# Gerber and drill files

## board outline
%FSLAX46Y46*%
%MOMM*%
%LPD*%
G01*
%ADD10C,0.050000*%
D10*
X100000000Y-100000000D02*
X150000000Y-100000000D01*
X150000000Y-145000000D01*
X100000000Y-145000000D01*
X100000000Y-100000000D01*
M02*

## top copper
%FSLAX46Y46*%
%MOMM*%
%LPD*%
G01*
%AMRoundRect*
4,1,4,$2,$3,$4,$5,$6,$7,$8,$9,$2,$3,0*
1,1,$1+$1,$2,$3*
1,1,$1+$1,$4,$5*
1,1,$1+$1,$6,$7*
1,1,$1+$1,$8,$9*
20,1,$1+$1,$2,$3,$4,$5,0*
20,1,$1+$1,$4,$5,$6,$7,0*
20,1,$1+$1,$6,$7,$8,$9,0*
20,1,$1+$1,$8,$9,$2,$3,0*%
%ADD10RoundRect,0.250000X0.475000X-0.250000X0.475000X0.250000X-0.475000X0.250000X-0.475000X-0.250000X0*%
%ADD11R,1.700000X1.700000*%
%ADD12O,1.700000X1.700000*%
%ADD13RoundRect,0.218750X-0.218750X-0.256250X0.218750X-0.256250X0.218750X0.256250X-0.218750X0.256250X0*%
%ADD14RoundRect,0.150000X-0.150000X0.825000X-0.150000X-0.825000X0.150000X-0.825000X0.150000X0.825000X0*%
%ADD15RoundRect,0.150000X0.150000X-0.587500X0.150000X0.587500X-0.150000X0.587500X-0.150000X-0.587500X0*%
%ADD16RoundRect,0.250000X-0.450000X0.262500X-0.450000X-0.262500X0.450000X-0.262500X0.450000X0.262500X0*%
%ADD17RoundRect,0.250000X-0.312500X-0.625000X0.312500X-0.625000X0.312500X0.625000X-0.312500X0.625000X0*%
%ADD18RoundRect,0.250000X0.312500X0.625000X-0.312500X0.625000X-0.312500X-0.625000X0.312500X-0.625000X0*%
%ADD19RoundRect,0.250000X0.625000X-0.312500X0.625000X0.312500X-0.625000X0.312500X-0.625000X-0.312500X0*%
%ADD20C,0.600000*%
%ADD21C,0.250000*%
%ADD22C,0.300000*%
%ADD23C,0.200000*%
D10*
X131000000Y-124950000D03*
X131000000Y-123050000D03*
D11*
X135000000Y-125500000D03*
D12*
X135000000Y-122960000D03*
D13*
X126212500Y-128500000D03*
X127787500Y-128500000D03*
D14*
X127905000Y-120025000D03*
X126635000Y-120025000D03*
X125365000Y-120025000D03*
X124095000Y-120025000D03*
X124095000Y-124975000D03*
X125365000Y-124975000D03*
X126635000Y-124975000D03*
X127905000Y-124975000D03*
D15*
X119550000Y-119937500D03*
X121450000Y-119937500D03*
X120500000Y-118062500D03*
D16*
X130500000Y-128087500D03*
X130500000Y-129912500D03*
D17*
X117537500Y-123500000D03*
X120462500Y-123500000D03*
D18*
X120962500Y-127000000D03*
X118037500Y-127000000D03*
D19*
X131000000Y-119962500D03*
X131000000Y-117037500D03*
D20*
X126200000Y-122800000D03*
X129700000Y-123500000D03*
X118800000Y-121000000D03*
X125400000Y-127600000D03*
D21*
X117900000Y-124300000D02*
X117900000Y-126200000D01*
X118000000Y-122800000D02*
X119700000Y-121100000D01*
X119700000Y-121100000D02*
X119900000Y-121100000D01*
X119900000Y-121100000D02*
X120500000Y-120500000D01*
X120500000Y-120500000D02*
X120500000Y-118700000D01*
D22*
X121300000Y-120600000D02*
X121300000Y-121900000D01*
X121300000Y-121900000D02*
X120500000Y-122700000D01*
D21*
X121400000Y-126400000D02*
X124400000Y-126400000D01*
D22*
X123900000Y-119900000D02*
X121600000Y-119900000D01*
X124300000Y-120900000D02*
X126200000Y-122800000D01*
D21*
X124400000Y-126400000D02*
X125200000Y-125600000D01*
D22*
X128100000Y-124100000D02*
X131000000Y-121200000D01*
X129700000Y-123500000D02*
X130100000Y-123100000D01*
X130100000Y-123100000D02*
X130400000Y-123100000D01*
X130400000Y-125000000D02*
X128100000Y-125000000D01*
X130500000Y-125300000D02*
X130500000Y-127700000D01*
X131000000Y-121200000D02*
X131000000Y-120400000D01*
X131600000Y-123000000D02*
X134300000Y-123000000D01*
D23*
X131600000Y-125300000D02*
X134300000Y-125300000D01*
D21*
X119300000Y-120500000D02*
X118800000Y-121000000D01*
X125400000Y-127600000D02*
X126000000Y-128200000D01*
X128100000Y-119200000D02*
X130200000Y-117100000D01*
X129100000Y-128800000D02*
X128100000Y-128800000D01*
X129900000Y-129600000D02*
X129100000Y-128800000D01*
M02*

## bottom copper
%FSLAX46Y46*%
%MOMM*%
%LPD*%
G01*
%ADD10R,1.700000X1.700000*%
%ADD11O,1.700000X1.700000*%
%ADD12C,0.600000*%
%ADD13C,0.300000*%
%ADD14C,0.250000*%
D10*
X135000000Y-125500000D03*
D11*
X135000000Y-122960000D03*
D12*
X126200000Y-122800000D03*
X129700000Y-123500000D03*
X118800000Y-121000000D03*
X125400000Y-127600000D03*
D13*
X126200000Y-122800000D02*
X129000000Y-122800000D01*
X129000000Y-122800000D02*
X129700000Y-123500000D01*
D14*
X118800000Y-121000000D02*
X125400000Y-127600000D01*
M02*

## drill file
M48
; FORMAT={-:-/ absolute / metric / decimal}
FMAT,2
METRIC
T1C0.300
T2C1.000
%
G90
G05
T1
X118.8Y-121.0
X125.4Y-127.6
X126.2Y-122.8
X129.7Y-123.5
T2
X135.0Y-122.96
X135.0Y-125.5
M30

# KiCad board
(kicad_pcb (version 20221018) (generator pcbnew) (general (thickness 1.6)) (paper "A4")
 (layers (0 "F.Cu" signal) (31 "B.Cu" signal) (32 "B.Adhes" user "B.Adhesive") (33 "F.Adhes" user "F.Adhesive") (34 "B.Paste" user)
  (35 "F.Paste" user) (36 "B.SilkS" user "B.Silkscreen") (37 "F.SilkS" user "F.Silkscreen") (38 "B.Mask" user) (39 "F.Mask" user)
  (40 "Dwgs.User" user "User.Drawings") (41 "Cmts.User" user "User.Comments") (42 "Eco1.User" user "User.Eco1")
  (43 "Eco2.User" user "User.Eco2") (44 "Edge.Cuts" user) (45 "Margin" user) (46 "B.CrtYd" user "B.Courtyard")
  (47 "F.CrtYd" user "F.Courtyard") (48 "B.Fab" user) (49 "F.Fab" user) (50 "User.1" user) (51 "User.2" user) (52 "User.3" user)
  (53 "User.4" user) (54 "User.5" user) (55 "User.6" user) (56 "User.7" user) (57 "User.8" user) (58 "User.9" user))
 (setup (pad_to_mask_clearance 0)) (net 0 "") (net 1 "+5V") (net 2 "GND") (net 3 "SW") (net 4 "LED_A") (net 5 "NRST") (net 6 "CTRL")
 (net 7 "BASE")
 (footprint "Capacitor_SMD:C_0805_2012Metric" (layer "F.Cu") (at 131 124 90)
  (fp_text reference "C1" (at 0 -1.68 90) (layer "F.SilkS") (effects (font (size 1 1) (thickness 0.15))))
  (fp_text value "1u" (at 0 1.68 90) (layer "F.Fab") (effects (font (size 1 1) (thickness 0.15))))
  (pad "1" smd roundrect (at -0.95 0 90) (size 1 1.45) (layers "F.Cu" "F.Paste" "F.Mask") (roundrect_rratio 0.25) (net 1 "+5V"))
  (pad "2" smd roundrect (at 0.95 0 90) (size 1 1.45) (layers "F.Cu" "F.Paste" "F.Mask") (roundrect_rratio 0.25) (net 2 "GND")))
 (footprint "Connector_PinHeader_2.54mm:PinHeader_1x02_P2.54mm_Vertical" (layer "F.Cu") (at 135 125.5 180)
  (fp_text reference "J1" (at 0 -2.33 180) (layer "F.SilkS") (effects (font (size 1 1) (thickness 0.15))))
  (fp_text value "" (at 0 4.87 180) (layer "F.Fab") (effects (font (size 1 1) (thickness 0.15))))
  (pad "1" thru_hole rect (at 0 0 180) (size 1.7 1.7) (drill 1) (layers "*.Cu" "*.Mask") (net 1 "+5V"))
  (pad "2" thru_hole oval (at 0 2.54 180) (size 1.7 1.7) (drill 1) (layers "*.Cu" "*.Mask") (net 2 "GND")))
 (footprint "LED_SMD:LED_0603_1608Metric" (layer "F.Cu") (at 127 128.5)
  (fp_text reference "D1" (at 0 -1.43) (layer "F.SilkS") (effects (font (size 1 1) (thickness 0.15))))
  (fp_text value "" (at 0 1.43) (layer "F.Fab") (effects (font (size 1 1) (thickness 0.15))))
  (pad "1" smd roundrect (at -0.7875 0) (size 0.875 0.95) (layers "F.Cu" "F.Paste" "F.Mask") (roundrect_rratio 0.25) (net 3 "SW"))
  (pad "2" smd roundrect (at 0.7875 0) (size 0.875 0.95) (layers "F.Cu" "F.Paste" "F.Mask") (roundrect_rratio 0.25) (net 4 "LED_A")))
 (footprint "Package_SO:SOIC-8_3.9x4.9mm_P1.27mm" (layer "F.Cu") (at 126 122.5 -90)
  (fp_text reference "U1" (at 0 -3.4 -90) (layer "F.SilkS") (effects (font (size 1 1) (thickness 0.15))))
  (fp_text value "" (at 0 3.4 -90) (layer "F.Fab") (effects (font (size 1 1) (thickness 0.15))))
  (pad "1" smd roundrect (at -2.475 -1.905 270) (size 1.95 0.6) (layers "F.Cu" "F.Paste" "F.Mask") (roundrect_rratio 0.25) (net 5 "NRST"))
  (pad "2" smd roundrect (at -2.475 -0.635 270) (size 1.95 0.6) (layers "F.Cu" "F.Paste" "F.Mask") (roundrect_rratio 0.25))
  (pad "3" smd roundrect (at -2.475 0.635 270) (size 1.95 0.6) (layers "F.Cu" "F.Paste" "F.Mask") (roundrect_rratio 0.25))
  (pad "4" smd roundrect (at -2.475 1.905 270) (size 1.95 0.6) (layers "F.Cu" "F.Paste" "F.Mask") (roundrect_rratio 0.25) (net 2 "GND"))
  (pad "5" smd roundrect (at 2.475 1.905 270) (size 1.95 0.6) (layers "F.Cu" "F.Paste" "F.Mask") (roundrect_rratio 0.25))
  (pad "6" smd roundrect (at 2.475 0.635 270) (size 1.95 0.6) (layers "F.Cu" "F.Paste" "F.Mask") (roundrect_rratio 0.25) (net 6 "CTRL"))
  (pad "7" smd roundrect (at 2.475 -0.635 270) (size 1.95 0.6) (layers "F.Cu" "F.Paste" "F.Mask") (roundrect_rratio 0.25))
  (pad "8" smd roundrect (at 2.475 -1.905 270) (size 1.95 0.6) (layers "F.Cu" "F.Paste" "F.Mask") (roundrect_rratio 0.25) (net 1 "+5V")))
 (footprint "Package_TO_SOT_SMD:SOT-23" (layer "F.Cu") (at 120.5 119 90)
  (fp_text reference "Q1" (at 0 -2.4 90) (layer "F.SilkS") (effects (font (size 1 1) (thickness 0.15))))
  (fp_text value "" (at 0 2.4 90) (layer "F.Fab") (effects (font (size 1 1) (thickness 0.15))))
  (pad "1" smd roundrect (at -0.9375 -0.95 90) (size 1.475 0.6) (layers "F.Cu" "F.Paste" "F.Mask") (roundrect_rratio 0.25) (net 3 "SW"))
  (pad "2" smd roundrect (at -0.9375 0.95 90) (size 1.475 0.6) (layers "F.Cu" "F.Paste" "F.Mask") (roundrect_rratio 0.25) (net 2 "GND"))
  (pad "3" smd roundrect (at 0.9375 0 90) (size 1.475 0.6) (layers "F.Cu" "F.Paste" "F.Mask") (roundrect_rratio 0.25) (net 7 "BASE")))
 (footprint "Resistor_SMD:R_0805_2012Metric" (layer "F.Cu") (at 130.5 129 -90)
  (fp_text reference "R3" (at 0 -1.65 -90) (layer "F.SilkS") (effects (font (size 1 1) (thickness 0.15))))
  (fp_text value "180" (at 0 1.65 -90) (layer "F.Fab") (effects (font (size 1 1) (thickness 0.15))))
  (pad "1" smd roundrect (at -0.9125 0 270) (size 1.025 1.4) (layers "F.Cu" "F.Paste" "F.Mask") (roundrect_rratio 0.243902) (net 1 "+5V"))
  (pad "2" smd roundrect (at 0.9125 0 270) (size 1.025 1.4) (layers "F.Cu" "F.Paste" "F.Mask") (roundrect_rratio 0.243902) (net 4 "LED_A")))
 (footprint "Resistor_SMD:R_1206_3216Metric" (layer "F.Cu") (at 119 123.5)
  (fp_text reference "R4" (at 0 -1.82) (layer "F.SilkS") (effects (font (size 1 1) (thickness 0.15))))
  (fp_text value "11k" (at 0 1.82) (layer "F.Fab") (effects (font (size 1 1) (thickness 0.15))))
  (pad "1" smd roundrect (at -1.4625 0) (size 1.125 1.75) (layers "F.Cu" "F.Paste" "F.Mask") (roundrect_rratio 0.222222) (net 7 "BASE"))
  (pad "2" smd roundrect (at 1.4625 0) (size 1.125 1.75) (layers "F.Cu" "F.Paste" "F.Mask") (roundrect_rratio 0.222222) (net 2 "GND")))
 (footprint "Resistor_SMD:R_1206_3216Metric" (layer "F.Cu") (at 119.5 127 180)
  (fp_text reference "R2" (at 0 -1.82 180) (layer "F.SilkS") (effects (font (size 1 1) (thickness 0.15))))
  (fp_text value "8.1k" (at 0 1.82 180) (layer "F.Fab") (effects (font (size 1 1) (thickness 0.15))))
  (pad "1" smd roundrect (at -1.4625 0 180) (size 1.125 1.75) (layers "F.Cu" "F.Paste" "F.Mask") (roundrect_rratio 0.222222) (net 6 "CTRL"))
  (pad "2" smd roundrect (at 1.4625 0 180) (size 1.125 1.75) (layers "F.Cu" "F.Paste" "F.Mask") (roundrect_rratio 0.222222) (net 7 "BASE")))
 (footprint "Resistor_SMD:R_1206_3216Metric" (layer "F.Cu") (at 131 118.5 90)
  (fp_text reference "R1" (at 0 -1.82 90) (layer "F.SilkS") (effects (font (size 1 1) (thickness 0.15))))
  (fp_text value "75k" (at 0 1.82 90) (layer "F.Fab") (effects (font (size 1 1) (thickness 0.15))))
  (pad "1" smd roundrect (at -1.4625 0 90) (size 1.125 1.75) (layers "F.Cu" "F.Paste" "F.Mask") (roundrect_rratio 0.222222) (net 1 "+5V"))
  (pad "2" smd roundrect (at 1.4625 0 90) (size 1.125 1.75) (layers "F.Cu" "F.Paste" "F.Mask") (roundrect_rratio 0.222222) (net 5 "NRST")))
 (gr_rect (start 100 100) (end 150 145) (stroke (width 0.05) (type default)) (fill none) (layer "Edge.Cuts"))
 (segment (start 117.9 124.3) (end 117.9 126.2) (width 0.25) (layer "F.Cu") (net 7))
 (segment (start 118 122.8) (end 119.7 121.1) (width 0.25) (layer "F.Cu") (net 7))
 (segment (start 119.7 121.1) (end 119.9 121.1) (width 0.25) (layer "F.Cu") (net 7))
 (segment (start 119.9 121.1) (end 120.5 120.5) (width 0.25) (layer "F.Cu") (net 7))
 (segment (start 120.5 120.5) (end 120.5 118.7) (width 0.25) (layer "F.Cu") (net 7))
 (segment (start 121.3 120.6) (end 121.3 121.9) (width 0.3) (layer "F.Cu") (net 2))
 (segment (start 121.3 121.9) (end 120.5 122.7) (width 0.3) (layer "F.Cu") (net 2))
 (segment (start 121.4 126.4) (end 124.4 126.4) (width 0.25) (layer "F.Cu") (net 6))
 (segment (start 123.9 119.9) (end 121.6 119.9) (width 0.3) (layer "F.Cu") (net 2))
 (segment (start 124.3 120.9) (end 126.2 122.8) (width 0.3) (layer "F.Cu") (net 2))
 (segment (start 124.4 126.4) (end 125.2 125.6) (width 0.25) (layer "F.Cu") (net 6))
 (segment (start 128.1 124.1) (end 131 121.2) (width 0.3) (layer "F.Cu") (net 1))
 (segment (start 129.7 123.5) (end 130.1 123.1) (width 0.3) (layer "F.Cu") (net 2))
 (segment (start 130.1 123.1) (end 130.4 123.1) (width 0.3) (layer "F.Cu") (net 2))
 (segment (start 130.4 125) (end 128.1 125) (width 0.3) (layer "F.Cu") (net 1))
 (segment (start 130.5 125.3) (end 130.5 127.7) (width 0.3) (layer "F.Cu") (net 1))
 (segment (start 131 121.2) (end 131 120.4) (width 0.3) (layer "F.Cu") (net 1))
 (segment (start 131.6 123) (end 134.3 123) (width 0.3) (layer "F.Cu") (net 2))
 (segment (start 131.6 125.3) (end 134.3 125.3) (width 0.2) (layer "F.Cu") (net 1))
 (via (at 126.2 122.8) (size 0.6) (drill 0.3) (layers "F.Cu" "B.Cu") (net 2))
 (via (at 129.7 123.5) (size 0.6) (drill 0.3) (layers "F.Cu" "B.Cu") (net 2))
 (segment (start 119.3 120.5) (end 118.8 121) (width 0.25) (layer "F.Cu") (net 3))
 (segment (start 125.4 127.6) (end 126 128.2) (width 0.25) (layer "F.Cu") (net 3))
 (segment (start 126.2 122.8) (end 129 122.8) (width 0.3) (layer "B.Cu") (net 2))
 (segment (start 128.1 119.2) (end 130.2 117.1) (width 0.25) (layer "F.Cu") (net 5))
 (segment (start 129 122.8) (end 129.7 123.5) (width 0.3) (layer "B.Cu") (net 2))
 (segment (start 129.1 128.8) (end 128.1 128.8) (width 0.25) (layer "F.Cu") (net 4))
 (segment (start 129.9 129.6) (end 129.1 128.8) (width 0.25) (layer "F.Cu") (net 4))
 (via (at 118.8 121) (size 0.6) (drill 0.3) (layers "F.Cu" "B.Cu") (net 3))
 (via (at 125.4 127.6) (size 0.6) (drill 0.3) (layers "F.Cu" "B.Cu") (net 3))
 (segment (start 118.8 121) (end 125.4 127.6) (width 0.25) (layer "B.Cu") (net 3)))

